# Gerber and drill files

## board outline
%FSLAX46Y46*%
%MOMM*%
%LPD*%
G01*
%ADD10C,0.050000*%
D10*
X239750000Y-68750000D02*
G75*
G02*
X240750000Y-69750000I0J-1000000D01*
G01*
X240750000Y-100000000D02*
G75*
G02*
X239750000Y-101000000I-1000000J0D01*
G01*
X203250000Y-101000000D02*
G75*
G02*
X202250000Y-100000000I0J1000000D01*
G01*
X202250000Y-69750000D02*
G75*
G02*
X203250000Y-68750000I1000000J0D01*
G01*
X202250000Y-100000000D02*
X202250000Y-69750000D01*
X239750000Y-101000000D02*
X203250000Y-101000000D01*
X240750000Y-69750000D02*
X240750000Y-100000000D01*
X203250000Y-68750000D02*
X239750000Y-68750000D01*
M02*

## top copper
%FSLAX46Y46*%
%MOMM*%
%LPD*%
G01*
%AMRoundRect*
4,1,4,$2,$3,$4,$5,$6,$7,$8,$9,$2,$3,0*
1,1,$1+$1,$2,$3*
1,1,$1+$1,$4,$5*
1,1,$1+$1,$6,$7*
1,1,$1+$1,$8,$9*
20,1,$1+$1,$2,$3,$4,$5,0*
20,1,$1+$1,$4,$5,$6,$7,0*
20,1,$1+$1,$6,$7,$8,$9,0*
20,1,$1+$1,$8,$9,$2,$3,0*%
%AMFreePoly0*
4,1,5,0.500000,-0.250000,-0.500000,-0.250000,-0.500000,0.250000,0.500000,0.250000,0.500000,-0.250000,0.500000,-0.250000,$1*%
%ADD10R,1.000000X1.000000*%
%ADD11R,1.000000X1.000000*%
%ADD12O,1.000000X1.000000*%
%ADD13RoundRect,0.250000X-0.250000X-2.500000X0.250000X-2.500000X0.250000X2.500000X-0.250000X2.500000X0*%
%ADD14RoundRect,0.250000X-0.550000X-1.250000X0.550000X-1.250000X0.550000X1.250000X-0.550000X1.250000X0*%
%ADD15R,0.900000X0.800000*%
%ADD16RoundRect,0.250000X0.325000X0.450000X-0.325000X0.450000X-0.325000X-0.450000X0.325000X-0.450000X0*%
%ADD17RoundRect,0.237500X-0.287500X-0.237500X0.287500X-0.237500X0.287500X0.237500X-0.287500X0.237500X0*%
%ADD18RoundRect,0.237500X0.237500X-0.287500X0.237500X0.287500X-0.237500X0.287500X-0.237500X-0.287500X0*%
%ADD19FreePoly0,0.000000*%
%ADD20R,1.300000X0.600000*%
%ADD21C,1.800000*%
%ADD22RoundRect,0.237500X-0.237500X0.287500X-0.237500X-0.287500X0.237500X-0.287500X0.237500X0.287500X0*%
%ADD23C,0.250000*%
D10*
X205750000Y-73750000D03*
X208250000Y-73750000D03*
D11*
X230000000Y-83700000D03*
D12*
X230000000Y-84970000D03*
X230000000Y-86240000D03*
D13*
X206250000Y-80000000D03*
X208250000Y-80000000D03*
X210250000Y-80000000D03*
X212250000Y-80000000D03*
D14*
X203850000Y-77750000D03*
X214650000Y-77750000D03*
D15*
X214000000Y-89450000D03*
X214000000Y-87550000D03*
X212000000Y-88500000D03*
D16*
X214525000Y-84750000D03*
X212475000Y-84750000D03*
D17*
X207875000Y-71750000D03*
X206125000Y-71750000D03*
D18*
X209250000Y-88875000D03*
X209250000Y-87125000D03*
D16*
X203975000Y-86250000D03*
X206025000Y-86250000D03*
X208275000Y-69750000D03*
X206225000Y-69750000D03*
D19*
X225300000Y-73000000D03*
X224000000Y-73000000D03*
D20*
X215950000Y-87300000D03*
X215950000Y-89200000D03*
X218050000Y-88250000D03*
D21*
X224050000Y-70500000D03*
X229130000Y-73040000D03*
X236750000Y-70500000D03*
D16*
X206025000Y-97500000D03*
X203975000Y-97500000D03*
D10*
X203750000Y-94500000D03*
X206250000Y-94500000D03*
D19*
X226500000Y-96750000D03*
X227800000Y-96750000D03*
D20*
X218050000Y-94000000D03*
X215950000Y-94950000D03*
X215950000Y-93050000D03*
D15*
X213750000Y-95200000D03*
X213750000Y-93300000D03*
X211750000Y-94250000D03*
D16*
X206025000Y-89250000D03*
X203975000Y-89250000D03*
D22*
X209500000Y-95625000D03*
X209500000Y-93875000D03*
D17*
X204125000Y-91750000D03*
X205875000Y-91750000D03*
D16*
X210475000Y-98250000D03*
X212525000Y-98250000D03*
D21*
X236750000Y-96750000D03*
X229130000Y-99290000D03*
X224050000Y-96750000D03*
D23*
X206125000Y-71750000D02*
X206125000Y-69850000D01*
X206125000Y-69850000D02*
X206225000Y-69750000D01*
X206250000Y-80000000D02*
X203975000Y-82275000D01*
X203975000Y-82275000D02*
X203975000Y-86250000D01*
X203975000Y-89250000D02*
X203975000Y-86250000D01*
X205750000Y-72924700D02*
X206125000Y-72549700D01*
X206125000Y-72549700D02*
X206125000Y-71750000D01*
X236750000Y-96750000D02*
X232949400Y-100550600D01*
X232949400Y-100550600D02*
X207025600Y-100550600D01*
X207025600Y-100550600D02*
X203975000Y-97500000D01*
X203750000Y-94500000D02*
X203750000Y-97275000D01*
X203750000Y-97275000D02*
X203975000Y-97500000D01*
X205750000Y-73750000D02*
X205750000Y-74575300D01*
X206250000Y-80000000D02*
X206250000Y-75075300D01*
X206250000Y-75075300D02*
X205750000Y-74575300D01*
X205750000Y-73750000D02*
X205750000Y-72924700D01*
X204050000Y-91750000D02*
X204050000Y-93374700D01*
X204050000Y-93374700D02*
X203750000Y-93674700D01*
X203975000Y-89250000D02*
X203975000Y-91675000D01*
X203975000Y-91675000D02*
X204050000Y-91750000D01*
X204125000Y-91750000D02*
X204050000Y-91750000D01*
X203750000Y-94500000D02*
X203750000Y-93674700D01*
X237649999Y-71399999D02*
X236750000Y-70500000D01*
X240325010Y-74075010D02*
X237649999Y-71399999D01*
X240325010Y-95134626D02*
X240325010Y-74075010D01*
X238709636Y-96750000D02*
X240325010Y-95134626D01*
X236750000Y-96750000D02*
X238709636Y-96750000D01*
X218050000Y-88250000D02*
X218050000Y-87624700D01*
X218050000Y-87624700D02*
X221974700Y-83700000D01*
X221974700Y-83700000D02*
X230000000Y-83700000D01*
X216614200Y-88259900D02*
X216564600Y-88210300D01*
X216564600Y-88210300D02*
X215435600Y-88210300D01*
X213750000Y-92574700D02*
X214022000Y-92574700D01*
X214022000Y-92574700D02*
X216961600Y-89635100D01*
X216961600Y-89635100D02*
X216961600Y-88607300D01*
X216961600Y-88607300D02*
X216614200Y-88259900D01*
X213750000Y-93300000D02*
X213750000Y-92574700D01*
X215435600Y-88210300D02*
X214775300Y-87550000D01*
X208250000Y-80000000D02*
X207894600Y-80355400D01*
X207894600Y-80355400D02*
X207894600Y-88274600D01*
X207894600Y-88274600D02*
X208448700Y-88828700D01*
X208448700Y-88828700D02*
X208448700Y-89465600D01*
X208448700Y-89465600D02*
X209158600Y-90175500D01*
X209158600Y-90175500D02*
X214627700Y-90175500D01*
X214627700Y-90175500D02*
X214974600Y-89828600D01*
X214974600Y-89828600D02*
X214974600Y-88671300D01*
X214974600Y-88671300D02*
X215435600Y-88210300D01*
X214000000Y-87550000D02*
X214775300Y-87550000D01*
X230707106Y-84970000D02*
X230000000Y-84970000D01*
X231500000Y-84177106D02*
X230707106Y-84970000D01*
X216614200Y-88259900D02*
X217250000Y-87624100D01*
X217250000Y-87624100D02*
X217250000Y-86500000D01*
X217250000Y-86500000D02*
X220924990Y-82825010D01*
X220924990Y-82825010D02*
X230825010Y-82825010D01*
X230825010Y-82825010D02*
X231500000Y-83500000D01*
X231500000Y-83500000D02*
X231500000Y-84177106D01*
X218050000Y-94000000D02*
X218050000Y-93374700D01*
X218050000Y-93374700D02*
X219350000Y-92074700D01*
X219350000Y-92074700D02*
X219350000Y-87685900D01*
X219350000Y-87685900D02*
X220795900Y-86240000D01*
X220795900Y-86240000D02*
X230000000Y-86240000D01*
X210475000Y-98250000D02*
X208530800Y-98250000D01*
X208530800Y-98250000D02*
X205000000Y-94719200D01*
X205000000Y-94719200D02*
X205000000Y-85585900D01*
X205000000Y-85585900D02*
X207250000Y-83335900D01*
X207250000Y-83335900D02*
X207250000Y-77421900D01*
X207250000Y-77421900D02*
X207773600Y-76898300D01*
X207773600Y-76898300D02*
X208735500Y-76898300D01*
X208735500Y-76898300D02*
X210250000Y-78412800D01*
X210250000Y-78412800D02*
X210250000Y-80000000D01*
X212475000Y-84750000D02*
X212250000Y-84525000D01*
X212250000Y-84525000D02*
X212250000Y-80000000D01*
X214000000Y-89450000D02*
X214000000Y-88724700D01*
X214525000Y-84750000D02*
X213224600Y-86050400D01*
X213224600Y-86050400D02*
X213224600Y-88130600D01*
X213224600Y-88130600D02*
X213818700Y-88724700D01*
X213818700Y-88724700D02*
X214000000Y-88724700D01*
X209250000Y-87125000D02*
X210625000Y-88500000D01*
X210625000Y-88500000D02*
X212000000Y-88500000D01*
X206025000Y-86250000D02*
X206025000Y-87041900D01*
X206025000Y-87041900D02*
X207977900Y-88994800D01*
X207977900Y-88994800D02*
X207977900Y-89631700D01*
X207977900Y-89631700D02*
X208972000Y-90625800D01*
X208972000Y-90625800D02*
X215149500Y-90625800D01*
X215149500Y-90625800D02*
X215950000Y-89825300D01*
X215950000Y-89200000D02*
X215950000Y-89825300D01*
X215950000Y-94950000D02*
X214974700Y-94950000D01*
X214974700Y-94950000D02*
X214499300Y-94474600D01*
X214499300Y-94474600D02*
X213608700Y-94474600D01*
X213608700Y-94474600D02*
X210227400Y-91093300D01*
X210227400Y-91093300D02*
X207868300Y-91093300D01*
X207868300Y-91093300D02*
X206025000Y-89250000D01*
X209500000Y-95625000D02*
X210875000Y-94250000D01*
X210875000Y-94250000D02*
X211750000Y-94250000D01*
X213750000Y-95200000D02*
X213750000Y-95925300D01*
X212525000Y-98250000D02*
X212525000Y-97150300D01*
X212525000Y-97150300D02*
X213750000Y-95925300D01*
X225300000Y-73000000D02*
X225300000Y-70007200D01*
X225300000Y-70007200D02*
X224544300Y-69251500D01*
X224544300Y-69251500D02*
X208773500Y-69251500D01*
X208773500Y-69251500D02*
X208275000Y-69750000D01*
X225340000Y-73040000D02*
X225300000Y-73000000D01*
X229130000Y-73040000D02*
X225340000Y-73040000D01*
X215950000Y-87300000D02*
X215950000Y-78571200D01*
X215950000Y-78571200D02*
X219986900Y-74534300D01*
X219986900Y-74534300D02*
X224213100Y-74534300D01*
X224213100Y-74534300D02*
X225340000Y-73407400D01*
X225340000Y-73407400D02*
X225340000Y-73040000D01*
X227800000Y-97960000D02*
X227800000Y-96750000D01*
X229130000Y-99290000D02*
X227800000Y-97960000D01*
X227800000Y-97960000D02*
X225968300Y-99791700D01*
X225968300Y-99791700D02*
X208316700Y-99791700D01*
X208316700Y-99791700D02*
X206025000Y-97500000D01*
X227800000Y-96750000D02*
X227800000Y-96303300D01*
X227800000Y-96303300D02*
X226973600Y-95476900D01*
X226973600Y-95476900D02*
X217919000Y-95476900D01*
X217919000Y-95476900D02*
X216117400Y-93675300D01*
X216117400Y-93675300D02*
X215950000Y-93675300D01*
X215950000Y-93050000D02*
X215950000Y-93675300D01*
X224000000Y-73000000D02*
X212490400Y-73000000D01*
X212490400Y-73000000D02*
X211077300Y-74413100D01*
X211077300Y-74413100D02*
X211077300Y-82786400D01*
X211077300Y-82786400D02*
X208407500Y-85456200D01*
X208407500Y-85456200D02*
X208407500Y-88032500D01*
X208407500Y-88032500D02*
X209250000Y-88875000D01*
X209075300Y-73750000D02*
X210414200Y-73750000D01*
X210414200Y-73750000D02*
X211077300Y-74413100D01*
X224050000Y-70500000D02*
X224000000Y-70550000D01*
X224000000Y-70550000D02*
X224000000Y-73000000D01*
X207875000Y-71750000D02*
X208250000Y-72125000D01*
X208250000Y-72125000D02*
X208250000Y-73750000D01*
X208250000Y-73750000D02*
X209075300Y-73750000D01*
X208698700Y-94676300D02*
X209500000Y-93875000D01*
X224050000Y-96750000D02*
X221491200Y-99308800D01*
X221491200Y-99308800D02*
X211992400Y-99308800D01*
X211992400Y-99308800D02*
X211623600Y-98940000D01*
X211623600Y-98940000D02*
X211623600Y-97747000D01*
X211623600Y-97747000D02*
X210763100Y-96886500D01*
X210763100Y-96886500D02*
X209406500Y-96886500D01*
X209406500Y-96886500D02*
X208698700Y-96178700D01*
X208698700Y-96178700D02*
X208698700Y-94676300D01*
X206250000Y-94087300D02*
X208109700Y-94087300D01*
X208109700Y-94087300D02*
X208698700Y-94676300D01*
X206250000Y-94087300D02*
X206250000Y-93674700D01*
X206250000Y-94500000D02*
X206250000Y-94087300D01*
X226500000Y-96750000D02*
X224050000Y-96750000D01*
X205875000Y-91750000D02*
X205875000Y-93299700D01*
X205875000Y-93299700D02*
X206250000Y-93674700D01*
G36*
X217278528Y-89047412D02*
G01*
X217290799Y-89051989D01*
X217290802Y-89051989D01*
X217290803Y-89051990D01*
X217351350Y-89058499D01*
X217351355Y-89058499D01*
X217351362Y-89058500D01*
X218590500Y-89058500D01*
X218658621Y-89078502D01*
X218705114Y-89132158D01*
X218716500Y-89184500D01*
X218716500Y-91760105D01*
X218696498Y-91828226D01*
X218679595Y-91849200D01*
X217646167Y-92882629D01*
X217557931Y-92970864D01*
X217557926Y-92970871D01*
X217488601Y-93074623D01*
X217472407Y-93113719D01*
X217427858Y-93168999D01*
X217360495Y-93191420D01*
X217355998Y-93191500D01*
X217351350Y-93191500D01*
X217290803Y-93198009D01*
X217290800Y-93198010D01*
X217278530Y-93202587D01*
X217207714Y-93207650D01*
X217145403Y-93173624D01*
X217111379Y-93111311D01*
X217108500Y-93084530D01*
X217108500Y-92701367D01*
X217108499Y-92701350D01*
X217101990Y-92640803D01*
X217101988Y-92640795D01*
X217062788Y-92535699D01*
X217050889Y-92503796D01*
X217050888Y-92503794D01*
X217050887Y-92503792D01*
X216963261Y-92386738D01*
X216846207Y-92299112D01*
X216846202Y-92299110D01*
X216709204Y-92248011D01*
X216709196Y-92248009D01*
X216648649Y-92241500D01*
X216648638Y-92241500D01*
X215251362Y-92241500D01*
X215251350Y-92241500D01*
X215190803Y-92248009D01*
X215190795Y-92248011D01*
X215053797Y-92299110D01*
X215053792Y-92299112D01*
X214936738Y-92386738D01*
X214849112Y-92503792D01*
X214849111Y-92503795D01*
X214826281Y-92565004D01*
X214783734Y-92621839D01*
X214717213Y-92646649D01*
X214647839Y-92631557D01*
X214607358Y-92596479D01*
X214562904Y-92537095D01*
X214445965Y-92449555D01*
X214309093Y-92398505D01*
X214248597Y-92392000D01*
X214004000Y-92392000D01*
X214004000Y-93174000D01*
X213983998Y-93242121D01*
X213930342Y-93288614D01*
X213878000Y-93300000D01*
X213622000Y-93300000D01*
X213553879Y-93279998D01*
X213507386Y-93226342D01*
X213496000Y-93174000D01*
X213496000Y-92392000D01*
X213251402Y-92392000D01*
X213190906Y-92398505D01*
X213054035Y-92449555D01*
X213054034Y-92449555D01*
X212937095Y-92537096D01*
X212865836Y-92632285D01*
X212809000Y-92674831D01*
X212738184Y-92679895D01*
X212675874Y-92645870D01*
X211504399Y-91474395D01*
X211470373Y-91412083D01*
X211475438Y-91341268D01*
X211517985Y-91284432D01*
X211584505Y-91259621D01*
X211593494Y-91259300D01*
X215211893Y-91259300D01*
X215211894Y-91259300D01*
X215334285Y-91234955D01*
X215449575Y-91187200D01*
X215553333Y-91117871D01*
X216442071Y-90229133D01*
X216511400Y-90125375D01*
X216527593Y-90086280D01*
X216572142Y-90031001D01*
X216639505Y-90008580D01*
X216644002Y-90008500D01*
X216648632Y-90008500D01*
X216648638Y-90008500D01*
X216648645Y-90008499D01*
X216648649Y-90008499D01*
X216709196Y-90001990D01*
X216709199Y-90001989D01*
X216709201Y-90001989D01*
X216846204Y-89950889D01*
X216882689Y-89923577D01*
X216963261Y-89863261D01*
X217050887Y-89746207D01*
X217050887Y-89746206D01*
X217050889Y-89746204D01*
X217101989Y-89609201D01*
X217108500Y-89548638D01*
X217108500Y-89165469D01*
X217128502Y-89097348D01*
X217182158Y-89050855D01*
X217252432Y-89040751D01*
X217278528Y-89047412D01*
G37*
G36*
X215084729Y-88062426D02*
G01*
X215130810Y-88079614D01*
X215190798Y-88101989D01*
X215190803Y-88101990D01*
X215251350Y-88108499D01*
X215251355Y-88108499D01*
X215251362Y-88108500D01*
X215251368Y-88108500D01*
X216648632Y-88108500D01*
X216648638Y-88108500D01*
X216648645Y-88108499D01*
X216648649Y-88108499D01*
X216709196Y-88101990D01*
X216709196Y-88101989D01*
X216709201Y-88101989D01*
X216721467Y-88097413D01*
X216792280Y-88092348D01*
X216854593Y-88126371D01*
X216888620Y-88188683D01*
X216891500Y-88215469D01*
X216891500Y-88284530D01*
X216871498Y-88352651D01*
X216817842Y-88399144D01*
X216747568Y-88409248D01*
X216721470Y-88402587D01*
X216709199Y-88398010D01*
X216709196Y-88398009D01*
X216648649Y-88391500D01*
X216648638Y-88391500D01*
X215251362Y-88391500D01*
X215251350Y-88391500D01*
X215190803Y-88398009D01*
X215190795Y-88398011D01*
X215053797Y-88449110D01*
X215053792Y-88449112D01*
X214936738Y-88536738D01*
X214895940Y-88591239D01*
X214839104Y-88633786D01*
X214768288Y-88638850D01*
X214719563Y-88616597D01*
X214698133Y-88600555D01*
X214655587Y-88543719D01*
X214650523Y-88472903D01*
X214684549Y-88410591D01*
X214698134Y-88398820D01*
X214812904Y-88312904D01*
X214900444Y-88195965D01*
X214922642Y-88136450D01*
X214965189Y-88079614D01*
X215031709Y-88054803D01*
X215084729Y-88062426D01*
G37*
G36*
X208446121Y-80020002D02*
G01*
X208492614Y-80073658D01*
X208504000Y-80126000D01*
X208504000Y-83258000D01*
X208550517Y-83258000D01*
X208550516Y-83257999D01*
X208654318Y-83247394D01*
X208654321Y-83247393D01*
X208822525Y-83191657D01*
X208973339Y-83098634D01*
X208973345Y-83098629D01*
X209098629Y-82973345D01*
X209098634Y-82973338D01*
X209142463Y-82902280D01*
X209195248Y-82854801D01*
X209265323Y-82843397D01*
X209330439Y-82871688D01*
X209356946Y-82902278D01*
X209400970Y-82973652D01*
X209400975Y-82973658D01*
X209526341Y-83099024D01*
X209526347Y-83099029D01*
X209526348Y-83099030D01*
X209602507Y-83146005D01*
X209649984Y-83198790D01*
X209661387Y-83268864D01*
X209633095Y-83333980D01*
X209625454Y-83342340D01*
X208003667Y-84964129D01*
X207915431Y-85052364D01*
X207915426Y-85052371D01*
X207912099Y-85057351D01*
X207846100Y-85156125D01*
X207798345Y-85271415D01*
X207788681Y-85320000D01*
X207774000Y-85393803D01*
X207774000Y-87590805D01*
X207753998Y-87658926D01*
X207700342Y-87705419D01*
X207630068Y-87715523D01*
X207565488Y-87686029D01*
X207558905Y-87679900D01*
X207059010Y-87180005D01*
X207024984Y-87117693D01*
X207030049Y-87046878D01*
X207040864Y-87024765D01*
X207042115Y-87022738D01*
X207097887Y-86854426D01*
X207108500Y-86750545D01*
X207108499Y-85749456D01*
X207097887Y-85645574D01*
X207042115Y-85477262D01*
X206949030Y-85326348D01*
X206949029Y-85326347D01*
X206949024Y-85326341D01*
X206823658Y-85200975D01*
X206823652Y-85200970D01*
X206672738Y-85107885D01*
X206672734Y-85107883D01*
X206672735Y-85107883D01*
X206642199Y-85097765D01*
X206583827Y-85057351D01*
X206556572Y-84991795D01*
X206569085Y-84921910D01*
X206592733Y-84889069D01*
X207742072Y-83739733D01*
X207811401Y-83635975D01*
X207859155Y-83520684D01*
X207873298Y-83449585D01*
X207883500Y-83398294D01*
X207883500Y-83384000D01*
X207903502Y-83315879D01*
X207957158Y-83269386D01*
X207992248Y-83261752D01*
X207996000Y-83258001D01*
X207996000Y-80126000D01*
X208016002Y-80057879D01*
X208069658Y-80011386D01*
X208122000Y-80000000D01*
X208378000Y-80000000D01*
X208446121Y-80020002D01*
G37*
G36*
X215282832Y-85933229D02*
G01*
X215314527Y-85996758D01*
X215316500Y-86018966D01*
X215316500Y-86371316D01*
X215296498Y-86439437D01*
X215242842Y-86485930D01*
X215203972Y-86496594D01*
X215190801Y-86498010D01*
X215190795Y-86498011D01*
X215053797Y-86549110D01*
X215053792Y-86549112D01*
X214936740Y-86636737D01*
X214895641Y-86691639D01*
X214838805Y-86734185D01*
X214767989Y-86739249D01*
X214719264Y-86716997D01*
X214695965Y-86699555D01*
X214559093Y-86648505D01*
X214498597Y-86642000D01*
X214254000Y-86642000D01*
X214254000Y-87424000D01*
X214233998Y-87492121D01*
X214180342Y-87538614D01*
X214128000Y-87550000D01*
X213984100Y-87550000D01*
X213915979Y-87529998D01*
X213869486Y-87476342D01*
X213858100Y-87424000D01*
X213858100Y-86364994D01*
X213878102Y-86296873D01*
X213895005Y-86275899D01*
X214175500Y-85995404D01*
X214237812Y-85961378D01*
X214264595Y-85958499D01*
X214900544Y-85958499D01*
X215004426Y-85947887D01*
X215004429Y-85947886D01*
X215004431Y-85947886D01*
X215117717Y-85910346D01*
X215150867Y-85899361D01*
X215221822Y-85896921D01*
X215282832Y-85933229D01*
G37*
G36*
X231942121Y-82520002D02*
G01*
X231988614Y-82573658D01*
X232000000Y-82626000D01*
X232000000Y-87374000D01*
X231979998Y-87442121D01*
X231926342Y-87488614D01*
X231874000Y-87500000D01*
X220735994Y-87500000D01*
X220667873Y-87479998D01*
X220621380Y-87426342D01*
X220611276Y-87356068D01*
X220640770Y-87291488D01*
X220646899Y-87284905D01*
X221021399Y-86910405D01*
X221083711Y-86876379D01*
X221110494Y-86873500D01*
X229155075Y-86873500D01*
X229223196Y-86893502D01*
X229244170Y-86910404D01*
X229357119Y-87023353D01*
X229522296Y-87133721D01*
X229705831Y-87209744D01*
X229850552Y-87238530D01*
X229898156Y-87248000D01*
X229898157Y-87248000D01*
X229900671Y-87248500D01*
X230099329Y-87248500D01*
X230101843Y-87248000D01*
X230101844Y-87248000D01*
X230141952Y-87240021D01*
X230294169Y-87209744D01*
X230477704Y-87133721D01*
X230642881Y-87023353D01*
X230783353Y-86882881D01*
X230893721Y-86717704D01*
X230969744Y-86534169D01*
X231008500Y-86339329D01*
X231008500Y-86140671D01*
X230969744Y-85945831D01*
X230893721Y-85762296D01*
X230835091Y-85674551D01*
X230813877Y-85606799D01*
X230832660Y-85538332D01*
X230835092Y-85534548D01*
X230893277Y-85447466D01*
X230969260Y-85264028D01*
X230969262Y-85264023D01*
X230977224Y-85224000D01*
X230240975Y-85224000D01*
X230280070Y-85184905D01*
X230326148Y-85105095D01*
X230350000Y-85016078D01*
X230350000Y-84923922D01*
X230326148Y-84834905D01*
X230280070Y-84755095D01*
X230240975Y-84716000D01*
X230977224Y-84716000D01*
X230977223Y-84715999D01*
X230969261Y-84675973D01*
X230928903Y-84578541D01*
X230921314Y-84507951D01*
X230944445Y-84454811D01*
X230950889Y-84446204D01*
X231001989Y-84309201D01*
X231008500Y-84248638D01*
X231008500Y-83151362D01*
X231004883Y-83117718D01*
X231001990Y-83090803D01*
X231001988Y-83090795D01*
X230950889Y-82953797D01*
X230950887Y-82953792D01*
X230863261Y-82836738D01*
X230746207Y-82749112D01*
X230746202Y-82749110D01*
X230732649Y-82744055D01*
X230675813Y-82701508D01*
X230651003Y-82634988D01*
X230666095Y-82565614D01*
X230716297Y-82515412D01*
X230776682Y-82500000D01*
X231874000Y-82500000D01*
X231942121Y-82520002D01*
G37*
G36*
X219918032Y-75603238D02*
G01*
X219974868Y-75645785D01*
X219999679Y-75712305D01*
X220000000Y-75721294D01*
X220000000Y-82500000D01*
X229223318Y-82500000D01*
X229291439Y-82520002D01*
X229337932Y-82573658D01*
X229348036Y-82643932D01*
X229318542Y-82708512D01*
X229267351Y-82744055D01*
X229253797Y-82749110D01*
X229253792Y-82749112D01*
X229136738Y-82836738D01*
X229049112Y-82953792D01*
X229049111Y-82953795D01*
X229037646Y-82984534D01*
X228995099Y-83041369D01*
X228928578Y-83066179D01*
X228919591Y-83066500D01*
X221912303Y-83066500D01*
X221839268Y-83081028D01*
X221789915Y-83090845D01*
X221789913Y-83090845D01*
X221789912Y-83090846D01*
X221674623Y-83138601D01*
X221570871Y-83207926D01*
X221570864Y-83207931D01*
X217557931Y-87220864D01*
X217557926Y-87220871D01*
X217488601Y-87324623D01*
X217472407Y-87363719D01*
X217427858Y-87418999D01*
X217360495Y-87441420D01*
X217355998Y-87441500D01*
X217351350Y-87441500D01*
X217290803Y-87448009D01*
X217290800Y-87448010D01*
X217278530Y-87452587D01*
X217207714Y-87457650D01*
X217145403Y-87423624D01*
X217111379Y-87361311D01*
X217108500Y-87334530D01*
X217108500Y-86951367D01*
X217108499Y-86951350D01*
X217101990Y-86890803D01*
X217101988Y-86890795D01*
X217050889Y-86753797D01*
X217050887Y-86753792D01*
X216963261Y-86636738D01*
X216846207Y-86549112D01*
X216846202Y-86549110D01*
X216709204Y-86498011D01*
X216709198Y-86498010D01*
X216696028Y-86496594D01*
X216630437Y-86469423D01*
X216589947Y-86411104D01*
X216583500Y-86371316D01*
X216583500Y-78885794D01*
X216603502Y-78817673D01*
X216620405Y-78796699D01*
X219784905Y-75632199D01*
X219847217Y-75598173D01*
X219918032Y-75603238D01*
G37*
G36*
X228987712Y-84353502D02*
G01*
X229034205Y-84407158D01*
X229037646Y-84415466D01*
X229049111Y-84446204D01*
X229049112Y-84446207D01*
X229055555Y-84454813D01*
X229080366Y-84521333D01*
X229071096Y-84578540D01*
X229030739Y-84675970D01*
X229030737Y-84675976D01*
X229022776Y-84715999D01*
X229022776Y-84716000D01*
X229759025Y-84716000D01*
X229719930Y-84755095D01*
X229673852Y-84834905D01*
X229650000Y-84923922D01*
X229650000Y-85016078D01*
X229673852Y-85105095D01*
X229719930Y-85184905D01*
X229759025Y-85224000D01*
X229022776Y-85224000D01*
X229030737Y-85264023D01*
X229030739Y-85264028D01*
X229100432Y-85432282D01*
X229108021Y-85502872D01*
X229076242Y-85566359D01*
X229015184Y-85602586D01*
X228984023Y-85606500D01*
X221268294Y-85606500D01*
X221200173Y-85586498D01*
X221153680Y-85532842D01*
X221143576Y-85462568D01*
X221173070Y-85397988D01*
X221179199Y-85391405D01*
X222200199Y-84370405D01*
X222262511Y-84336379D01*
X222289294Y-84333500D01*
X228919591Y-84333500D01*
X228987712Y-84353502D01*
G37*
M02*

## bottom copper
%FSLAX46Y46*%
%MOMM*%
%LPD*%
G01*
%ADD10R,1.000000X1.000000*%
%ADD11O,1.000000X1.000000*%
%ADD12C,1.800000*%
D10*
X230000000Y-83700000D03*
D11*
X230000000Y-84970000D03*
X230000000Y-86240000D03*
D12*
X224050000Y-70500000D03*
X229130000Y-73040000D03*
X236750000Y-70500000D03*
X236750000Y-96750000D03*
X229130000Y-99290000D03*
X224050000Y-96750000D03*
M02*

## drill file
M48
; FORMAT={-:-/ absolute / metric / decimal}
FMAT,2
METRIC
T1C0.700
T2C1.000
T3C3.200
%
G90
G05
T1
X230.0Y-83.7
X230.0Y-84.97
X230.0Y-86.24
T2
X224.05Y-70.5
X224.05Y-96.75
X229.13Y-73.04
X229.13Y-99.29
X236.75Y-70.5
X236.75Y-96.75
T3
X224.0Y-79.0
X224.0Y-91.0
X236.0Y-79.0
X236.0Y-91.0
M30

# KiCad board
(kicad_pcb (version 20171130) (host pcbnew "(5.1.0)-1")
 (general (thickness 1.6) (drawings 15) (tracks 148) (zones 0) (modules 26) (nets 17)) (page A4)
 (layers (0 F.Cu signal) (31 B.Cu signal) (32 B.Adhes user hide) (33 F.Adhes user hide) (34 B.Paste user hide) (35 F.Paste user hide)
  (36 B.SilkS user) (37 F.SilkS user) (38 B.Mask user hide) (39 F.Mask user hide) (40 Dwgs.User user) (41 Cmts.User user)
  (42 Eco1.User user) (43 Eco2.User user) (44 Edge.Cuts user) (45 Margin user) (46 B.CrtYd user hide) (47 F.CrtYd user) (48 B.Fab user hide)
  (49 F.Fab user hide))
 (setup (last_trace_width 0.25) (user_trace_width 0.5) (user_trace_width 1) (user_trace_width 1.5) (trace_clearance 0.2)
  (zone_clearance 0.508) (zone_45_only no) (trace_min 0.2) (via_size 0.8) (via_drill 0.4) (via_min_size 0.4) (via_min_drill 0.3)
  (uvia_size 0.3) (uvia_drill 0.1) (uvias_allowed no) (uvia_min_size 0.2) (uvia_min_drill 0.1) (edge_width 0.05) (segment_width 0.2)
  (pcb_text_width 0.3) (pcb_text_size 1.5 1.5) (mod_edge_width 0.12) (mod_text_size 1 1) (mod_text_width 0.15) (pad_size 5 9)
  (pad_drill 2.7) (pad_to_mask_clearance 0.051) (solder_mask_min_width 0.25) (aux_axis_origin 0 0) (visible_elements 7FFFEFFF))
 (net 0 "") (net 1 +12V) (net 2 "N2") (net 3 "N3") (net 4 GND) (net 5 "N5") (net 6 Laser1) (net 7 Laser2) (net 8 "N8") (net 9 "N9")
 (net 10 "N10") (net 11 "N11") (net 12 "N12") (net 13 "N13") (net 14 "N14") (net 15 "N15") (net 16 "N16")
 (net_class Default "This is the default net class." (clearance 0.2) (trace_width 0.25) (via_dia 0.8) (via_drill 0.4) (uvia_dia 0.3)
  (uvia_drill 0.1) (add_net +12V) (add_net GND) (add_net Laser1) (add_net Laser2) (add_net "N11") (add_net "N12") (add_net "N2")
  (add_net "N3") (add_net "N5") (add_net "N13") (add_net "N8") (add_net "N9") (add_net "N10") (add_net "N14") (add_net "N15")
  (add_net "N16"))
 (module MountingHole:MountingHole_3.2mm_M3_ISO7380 (layer F.Cu) (at 224 79)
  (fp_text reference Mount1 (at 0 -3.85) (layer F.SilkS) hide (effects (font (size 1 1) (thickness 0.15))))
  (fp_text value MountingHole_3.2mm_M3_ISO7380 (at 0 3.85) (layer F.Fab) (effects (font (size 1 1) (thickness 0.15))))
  (pad 1 np_thru_hole circle (at 0 0) (size 3.2 3.2) (drill 3.2) (layers *.Cu *.Mask)))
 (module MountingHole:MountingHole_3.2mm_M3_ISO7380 (layer F.Cu) (at 236 79)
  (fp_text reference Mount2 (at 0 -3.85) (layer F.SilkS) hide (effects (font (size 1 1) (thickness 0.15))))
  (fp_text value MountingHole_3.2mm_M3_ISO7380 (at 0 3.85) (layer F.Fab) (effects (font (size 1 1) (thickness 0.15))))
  (pad 1 np_thru_hole circle (at 0 0) (size 3.2 3.2) (drill 3.2) (layers *.Cu *.Mask)))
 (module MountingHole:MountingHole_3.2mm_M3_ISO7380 (layer F.Cu) (at 236 91)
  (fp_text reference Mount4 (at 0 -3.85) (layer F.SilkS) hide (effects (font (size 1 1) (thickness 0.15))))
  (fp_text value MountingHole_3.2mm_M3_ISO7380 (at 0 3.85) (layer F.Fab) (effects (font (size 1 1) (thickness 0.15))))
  (pad 1 np_thru_hole circle (at 0 0) (size 3.2 3.2) (drill 3.2) (layers *.Cu *.Mask)))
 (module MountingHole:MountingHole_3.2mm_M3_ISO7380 (layer F.Cu) (at 224 91)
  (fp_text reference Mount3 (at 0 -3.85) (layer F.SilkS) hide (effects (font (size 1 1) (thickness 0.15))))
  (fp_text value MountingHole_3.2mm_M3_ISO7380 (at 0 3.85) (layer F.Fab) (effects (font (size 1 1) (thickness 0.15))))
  (pad 1 np_thru_hole circle (at 0 0) (size 3.2 3.2) (drill 3.2) (layers *.Cu *.Mask)))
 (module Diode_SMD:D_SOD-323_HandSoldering (layer F.Cu) (at 207 73.75)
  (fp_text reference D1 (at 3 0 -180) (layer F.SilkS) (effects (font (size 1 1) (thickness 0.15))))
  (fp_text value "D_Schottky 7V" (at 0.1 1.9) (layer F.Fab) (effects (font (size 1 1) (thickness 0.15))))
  (pad 1 smd rect (at -1.25 0) (size 1 1) (layers F.Cu F.Paste F.Mask) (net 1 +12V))
  (pad 2 smd rect (at 1.25 0) (size 1 1) (layers F.Cu F.Paste F.Mask) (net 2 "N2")))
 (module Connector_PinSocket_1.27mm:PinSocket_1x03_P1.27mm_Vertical (layer F.Cu) (at 230 83.7)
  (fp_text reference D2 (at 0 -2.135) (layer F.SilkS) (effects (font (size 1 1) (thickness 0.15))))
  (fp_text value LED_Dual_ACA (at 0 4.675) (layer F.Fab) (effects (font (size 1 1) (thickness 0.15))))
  (pad 1 thru_hole rect (at 0 0) (size 1 1) (drill 0.7) (layers *.Cu *.Mask) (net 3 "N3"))
  (pad 2 thru_hole oval (at 0 1.27) (size 1 1) (drill 0.7) (layers *.Cu *.Mask) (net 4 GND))
  (pad 3 thru_hole oval (at 0 2.54) (size 1 1) (drill 0.7) (layers *.Cu *.Mask) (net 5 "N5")))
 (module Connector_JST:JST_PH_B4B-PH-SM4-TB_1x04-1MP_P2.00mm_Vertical (layer F.Cu) (at 209.25 79.5)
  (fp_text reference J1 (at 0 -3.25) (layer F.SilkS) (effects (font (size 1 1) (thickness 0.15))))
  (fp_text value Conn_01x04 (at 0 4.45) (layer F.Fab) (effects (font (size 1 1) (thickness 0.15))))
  (pad 1 smd roundrect (at -3 0.5) (size 1 5.5) (layers F.Cu F.Paste F.Mask) (roundrect_rratio 0.25) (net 1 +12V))
  (pad 2 smd roundrect (at -1 0.5) (size 1 5.5) (layers F.Cu F.Paste F.Mask) (roundrect_rratio 0.25) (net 4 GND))
  (pad 3 smd roundrect (at 1 0.5) (size 1 5.5) (layers F.Cu F.Paste F.Mask) (roundrect_rratio 0.25) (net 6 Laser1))
  (pad 4 smd roundrect (at 3 0.5) (size 1 5.5) (layers F.Cu F.Paste F.Mask) (roundrect_rratio 0.25) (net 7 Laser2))
  (pad MP smd roundrect (at -5.4 -1.75) (size 1.6 3) (layers F.Cu F.Paste F.Mask) (roundrect_rratio 0.15625))
  (pad MP smd roundrect (at 5.4 -1.75) (size 1.6 3) (layers F.Cu F.Paste F.Mask) (roundrect_rratio 0.15625)))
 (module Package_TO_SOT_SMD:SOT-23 (layer F.Cu) (at 213 88.5 180)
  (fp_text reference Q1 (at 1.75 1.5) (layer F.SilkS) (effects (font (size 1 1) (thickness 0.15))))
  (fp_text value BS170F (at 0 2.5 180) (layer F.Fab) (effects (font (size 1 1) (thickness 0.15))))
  (pad 1 smd rect (at -1 -0.95 180) (size 0.9 0.8) (layers F.Cu F.Paste F.Mask) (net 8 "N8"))
  (pad 2 smd rect (at -1 0.95 180) (size 0.9 0.8) (layers F.Cu F.Paste F.Mask) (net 4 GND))
  (pad 3 smd rect (at 1 0 180) (size 0.9 0.8) (layers F.Cu F.Paste F.Mask) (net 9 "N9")))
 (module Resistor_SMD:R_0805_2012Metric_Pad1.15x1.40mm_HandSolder (layer F.Cu) (at 213.5 84.75 180)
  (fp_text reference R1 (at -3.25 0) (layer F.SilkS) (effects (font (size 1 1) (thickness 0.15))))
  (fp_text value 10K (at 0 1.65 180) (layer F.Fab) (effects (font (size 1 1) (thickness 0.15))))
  (pad 1 smd roundrect (at -1.025 0 180) (size 1.15 1.4) (layers F.Cu F.Paste F.Mask) (roundrect_rratio 0.217391) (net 8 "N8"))
  (pad 2 smd roundrect (at 1.025 0 180) (size 1.15 1.4) (layers F.Cu F.Paste F.Mask) (roundrect_rratio 0.217391) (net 7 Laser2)))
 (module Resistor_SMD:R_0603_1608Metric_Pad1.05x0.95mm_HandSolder (layer F.Cu) (at 207 71.75)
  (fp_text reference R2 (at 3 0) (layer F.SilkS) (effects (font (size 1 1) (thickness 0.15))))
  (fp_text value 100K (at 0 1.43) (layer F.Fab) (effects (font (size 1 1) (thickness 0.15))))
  (pad 2 smd roundrect (at 0.875 0) (size 1.05 0.95) (layers F.Cu F.Paste F.Mask) (roundrect_rratio 0.25) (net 2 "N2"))
  (pad 1 smd roundrect (at -0.875 0) (size 1.05 0.95) (layers F.Cu F.Paste F.Mask) (roundrect_rratio 0.25) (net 1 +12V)))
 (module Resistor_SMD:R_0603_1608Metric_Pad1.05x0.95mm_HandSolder (layer F.Cu) (at 209.25 88 90)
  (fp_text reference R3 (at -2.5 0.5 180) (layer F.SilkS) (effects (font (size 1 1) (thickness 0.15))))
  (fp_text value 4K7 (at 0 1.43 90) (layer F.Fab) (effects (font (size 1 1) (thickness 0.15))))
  (pad 1 smd roundrect (at -0.875 0 90) (size 1.05 0.95) (layers F.Cu F.Paste F.Mask) (roundrect_rratio 0.25) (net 2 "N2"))
  (pad 2 smd roundrect (at 0.875 0 90) (size 1.05 0.95) (layers F.Cu F.Paste F.Mask) (roundrect_rratio 0.25) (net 9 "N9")))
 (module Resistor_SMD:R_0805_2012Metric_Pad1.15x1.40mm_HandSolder (layer F.Cu) (at 205 86.25 180)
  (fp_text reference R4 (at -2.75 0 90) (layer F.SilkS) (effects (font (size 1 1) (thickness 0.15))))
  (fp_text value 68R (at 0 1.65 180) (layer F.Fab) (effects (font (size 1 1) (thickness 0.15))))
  (pad 2 smd roundrect (at 1.025 0 180) (size 1.15 1.4) (layers F.Cu F.Paste F.Mask) (roundrect_rratio 0.217391) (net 1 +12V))
  (pad 1 smd roundrect (at -1.025 0 180) (size 1.15 1.4) (layers F.Cu F.Paste F.Mask) (roundrect_rratio 0.217391) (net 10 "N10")))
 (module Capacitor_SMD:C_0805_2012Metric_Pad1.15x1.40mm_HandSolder (layer F.Cu) (at 207.25 69.75 180)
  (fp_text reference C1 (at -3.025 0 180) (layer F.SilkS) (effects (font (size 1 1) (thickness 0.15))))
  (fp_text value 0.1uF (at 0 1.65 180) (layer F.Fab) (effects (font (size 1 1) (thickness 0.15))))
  (pad 1 smd roundrect (at -1.025 0 180) (size 1.15 1.4) (layers F.Cu F.Paste F.Mask) (roundrect_rratio 0.217391) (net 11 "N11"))
  (pad 2 smd roundrect (at 1.025 0 180) (size 1.15 1.4) (layers F.Cu F.Paste F.Mask) (roundrect_rratio 0.217391) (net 1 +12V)))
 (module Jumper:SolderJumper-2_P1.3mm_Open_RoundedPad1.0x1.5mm (layer F.Cu) (at 224.65 73)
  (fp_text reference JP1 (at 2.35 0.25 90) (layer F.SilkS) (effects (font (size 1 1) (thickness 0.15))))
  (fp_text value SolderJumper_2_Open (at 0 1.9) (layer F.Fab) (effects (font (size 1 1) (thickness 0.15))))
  (pad 2 smd custom (at 0.65 0) (size 1 0.5) (layers F.Cu F.Mask) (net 11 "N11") (zone_connect 2)
   (options (clearance outline) (anchor rect)) (primitives))
  (pad 1 smd custom (at -0.65 0) (size 1 0.5) (layers F.Cu F.Mask) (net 2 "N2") (zone_connect 2) (options (clearance outline) (anchor rect))
   (primitives)))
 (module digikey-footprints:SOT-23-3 (layer F.Cu) (at 217 88.25)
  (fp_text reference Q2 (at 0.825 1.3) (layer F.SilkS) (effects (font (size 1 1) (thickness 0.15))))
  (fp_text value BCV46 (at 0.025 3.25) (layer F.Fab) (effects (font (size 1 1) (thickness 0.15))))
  (pad 1 smd rect (at -1.05 -0.95) (size 1.3 0.6) (layers F.Cu F.Paste F.Mask) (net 11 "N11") (solder_mask_margin 0.07))
  (pad 2 smd rect (at -1.05 0.95) (size 1.3 0.6) (layers F.Cu F.Paste F.Mask) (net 10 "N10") (solder_mask_margin 0.07))
  (pad 3 smd rect (at 1.05 0) (size 1.3 0.6) (layers F.Cu F.Paste F.Mask) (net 3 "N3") (solder_mask_margin 0.07)))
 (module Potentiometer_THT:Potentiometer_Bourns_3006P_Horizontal (layer B.Cu) (at 236.75 70.5)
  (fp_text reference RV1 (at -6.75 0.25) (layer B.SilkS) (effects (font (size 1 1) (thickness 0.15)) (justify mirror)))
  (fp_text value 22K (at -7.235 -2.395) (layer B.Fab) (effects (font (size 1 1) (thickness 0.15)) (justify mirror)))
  (pad 3 thru_hole circle (at -12.7 0) (size 1.8 1.8) (drill 1) (layers *.Cu *.Mask) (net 2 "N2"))
  (pad 2 thru_hole circle (at -7.62 2.54) (size 1.8 1.8) (drill 1) (layers *.Cu *.Mask) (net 11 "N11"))
  (pad 1 thru_hole circle (at 0 0) (size 1.8 1.8) (drill 1) (layers *.Cu *.Mask) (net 1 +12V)))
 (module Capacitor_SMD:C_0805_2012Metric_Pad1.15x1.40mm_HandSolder (layer F.Cu) (at 205 97.5 180)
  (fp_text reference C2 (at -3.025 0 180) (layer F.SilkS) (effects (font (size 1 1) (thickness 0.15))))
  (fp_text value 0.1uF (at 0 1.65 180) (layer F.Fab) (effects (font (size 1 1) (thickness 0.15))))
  (pad 1 smd roundrect (at -1.025 0 180) (size 1.15 1.4) (layers F.Cu F.Paste F.Mask) (roundrect_rratio 0.217391) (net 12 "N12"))
  (pad 2 smd roundrect (at 1.025 0 180) (size 1.15 1.4) (layers F.Cu F.Paste F.Mask) (roundrect_rratio 0.217391) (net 1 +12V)))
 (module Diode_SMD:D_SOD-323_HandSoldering (layer F.Cu) (at 205 94.5)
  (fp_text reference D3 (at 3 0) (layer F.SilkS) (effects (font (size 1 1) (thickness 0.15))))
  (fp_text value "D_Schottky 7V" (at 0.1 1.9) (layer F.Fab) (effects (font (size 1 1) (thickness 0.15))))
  (pad 1 smd rect (at -1.25 0) (size 1 1) (layers F.Cu F.Paste F.Mask) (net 1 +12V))
  (pad 2 smd rect (at 1.25 0) (size 1 1) (layers F.Cu F.Paste F.Mask) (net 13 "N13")))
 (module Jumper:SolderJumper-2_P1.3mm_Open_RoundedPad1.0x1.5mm (layer F.Cu) (at 227.15 96.75)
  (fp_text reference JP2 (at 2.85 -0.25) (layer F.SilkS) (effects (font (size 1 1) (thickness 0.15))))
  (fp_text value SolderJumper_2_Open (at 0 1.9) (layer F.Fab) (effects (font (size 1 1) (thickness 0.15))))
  (pad 1 smd custom (at -0.65 0) (size 1 0.5) (layers F.Cu F.Mask) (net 13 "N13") (zone_connect 2)
   (options (clearance outline) (anchor rect)) (primitives))
  (pad 2 smd custom (at 0.65 0) (size 1 0.5) (layers F.Cu F.Mask) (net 12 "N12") (zone_connect 2)
   (options (clearance outline) (anchor rect)) (primitives)))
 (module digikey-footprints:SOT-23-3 (layer F.Cu) (at 217 94)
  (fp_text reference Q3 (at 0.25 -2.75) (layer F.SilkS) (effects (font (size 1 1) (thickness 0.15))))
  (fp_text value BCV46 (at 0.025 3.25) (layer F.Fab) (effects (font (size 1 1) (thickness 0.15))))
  (pad 3 smd rect (at 1.05 0) (size 1.3 0.6) (layers F.Cu F.Paste F.Mask) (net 5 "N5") (solder_mask_margin 0.07))
  (pad 2 smd rect (at -1.05 0.95) (size 1.3 0.6) (layers F.Cu F.Paste F.Mask) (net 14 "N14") (solder_mask_margin 0.07))
  (pad 1 smd rect (at -1.05 -0.95) (size 1.3 0.6) (layers F.Cu F.Paste F.Mask) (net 12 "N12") (solder_mask_margin 0.07)))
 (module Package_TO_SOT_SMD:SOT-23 (layer F.Cu) (at 212.75 94.25 180)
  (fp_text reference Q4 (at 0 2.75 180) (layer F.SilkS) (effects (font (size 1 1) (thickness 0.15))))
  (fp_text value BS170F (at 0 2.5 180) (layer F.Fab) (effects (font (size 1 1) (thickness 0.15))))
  (pad 1 smd rect (at -1 -0.95 180) (size 0.9 0.8) (layers F.Cu F.Paste F.Mask) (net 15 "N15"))
  (pad 2 smd rect (at -1 0.95 180) (size 0.9 0.8) (layers F.Cu F.Paste F.Mask) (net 4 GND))
  (pad 3 smd rect (at 1 0 180) (size 0.9 0.8) (layers F.Cu F.Paste F.Mask) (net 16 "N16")))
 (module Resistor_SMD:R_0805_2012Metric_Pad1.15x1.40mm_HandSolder (layer F.Cu) (at 205 89.25 180)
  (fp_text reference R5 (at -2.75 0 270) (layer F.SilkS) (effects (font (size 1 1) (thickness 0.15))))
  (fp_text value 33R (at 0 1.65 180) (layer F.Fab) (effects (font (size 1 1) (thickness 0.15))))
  (pad 1 smd roundrect (at -1.025 0 180) (size 1.15 1.4) (layers F.Cu F.Paste F.Mask) (roundrect_rratio 0.217391) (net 14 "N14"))
  (pad 2 smd roundrect (at 1.025 0 180) (size 1.15 1.4) (layers F.Cu F.Paste F.Mask) (roundrect_rratio 0.217391) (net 1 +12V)))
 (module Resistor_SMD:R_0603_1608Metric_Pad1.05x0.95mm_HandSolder (layer F.Cu) (at 209.5 94.75 270)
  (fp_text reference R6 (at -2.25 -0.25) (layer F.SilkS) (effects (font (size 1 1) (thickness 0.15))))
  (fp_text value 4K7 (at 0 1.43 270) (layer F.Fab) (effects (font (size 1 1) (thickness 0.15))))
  (pad 2 smd roundrect (at 0.875 0 270) (size 1.05 0.95) (layers F.Cu F.Paste F.Mask) (roundrect_rratio 0.25) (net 16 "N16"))
  (pad 1 smd roundrect (at -0.875 0 270) (size 1.05 0.95) (layers F.Cu F.Paste F.Mask) (roundrect_rratio 0.25) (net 13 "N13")))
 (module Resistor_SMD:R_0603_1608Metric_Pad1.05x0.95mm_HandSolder (layer F.Cu) (at 205 91.75)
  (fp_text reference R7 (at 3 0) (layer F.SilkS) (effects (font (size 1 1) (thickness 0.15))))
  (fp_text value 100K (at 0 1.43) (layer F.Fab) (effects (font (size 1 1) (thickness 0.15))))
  (pad 1 smd roundrect (at -0.875 0) (size 1.05 0.95) (layers F.Cu F.Paste F.Mask) (roundrect_rratio 0.25) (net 1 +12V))
  (pad 2 smd roundrect (at 0.875 0) (size 1.05 0.95) (layers F.Cu F.Paste F.Mask) (roundrect_rratio 0.25) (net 13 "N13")))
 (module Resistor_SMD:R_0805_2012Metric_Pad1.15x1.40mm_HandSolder (layer F.Cu) (at 211.5 98.25 180)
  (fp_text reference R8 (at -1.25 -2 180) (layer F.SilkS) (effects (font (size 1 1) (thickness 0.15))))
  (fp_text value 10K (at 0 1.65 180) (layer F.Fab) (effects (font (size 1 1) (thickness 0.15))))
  (pad 2 smd roundrect (at 1.025 0 180) (size 1.15 1.4) (layers F.Cu F.Paste F.Mask) (roundrect_rratio 0.217391) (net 6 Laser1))
  (pad 1 smd roundrect (at -1.025 0 180) (size 1.15 1.4) (layers F.Cu F.Paste F.Mask) (roundrect_rratio 0.217391) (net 15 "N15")))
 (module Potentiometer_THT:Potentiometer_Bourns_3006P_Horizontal (layer B.Cu) (at 236.75 96.75)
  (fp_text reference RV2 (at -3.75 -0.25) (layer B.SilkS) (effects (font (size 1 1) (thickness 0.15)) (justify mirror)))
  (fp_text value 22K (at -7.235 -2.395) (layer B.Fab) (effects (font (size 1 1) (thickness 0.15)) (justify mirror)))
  (pad 1 thru_hole circle (at 0 0) (size 1.8 1.8) (drill 1) (layers *.Cu *.Mask) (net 1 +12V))
  (pad 2 thru_hole circle (at -7.62 2.54) (size 1.8 1.8) (drill 1) (layers *.Cu *.Mask) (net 12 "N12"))
  (pad 3 thru_hole circle (at -12.7 0) (size 1.8 1.8) (drill 1) (layers *.Cu *.Mask) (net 13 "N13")))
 (gr_arc (start 239.75 69.75) (end 240.75 69.75) (angle -90) (layer Edge.Cuts) (width 0.05))
 (gr_arc (start 239.75 100) (end 239.75 101) (angle -90) (layer Edge.Cuts) (width 0.05))
 (gr_arc (start 203.25 100) (end 202.25 100) (angle -90) (layer Edge.Cuts) (width 0.05))
 (gr_arc (start 203.25 69.75) (end 203.25 68.75) (angle -90) (layer Edge.Cuts) (width 0.05))
 (gr_line (start 202.25 100) (end 202.25 69.75) (layer Edge.Cuts) (width 0.05))
 (gr_line (start 239.75 101) (end 203.25 101) (layer Edge.Cuts) (width 0.05))
 (gr_line (start 240.75 69.75) (end 240.75 100) (layer Edge.Cuts) (width 0.05))
 (gr_line (start 203.25 68.75) (end 239.75 68.75) (layer Edge.Cuts) (width 0.05))
 (segment (start 206.125 71.75) (end 206.125 69.85) (width 0.25) (layer F.Cu) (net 1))
 (segment (start 206.125 69.85) (end 206.225 69.75) (width 0.25) (layer F.Cu) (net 1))
 (segment (start 206.25 80) (end 203.975 82.275) (width 0.25) (layer F.Cu) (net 1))
 (segment (start 203.975 82.275) (end 203.975 86.25) (width 0.25) (layer F.Cu) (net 1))
 (segment (start 203.975 89.25) (end 203.975 86.25) (width 0.25) (layer F.Cu) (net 1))
 (segment (start 205.75 72.9247) (end 206.125 72.5497) (width 0.25) (layer F.Cu) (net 1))
 (segment (start 206.125 72.5497) (end 206.125 71.75) (width 0.25) (layer F.Cu) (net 1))
 (segment (start 236.75 96.75) (end 232.9494 100.5506) (width 0.25) (layer F.Cu) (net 1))
 (segment (start 232.9494 100.5506) (end 207.0256 100.5506) (width 0.25) (layer F.Cu) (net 1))
 (segment (start 207.0256 100.5506) (end 203.975 97.5) (width 0.25) (layer F.Cu) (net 1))
 (segment (start 203.75 94.5) (end 203.75 97.275) (width 0.25) (layer F.Cu) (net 1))
 (segment (start 203.75 97.275) (end 203.975 97.5) (width 0.25) (layer F.Cu) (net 1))
 (segment (start 205.75 73.75) (end 205.75 74.5753) (width 0.25) (layer F.Cu) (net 1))
 (segment (start 206.25 80) (end 206.25 75.0753) (width 0.25) (layer F.Cu) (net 1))
 (segment (start 206.25 75.0753) (end 205.75 74.5753) (width 0.25) (layer F.Cu) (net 1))
 (segment (start 205.75 73.75) (end 205.75 72.9247) (width 0.25) (layer F.Cu) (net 1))
 (segment (start 204.05 91.75) (end 204.05 93.3747) (width 0.25) (layer F.Cu) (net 1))
 (segment (start 204.05 93.3747) (end 203.75 93.6747) (width 0.25) (layer F.Cu) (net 1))
 (segment (start 203.975 89.25) (end 203.975 91.675) (width 0.25) (layer F.Cu) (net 1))
 (segment (start 203.975 91.675) (end 204.05 91.75) (width 0.25) (layer F.Cu) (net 1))
 (segment (start 204.125 91.75) (end 204.05 91.75) (width 0.25) (layer F.Cu) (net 1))
 (segment (start 203.75 94.5) (end 203.75 93.6747) (width 0.25) (layer F.Cu) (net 1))
 (segment (start 237.649999 71.399999) (end 236.75 70.5) (width 0.25) (layer F.Cu) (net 1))
 (segment (start 240.32501 74.07501) (end 237.649999 71.399999) (width 0.25) (layer F.Cu) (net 1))
 (segment (start 240.32501 95.134626) (end 240.32501 74.07501) (width 0.25) (layer F.Cu) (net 1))
 (segment (start 238.709636 96.75) (end 240.32501 95.134626) (width 0.25) (layer F.Cu) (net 1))
 (segment (start 236.75 96.75) (end 238.709636 96.75) (width 0.25) (layer F.Cu) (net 1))
 (segment (start 218.05 88.25) (end 218.05 87.6247) (width 0.25) (layer F.Cu) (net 3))
 (segment (start 218.05 87.6247) (end 221.9747 83.7) (width 0.25) (layer F.Cu) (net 3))
 (segment (start 221.9747 83.7) (end 230 83.7) (width 0.25) (layer F.Cu) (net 3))
 (segment (start 216.6142 88.2599) (end 216.5646 88.2103) (width 0.25) (layer F.Cu) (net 4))
 (segment (start 216.5646 88.2103) (end 215.4356 88.2103) (width 0.25) (layer F.Cu) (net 4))
 (segment (start 213.75 92.5747) (end 214.022 92.5747) (width 0.25) (layer F.Cu) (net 4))
 (segment (start 214.022 92.5747) (end 216.9616 89.6351) (width 0.25) (layer F.Cu) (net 4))
 (segment (start 216.9616 89.6351) (end 216.9616 88.6073) (width 0.25) (layer F.Cu) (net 4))
 (segment (start 216.9616 88.6073) (end 216.6142 88.2599) (width 0.25) (layer F.Cu) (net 4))
 (segment (start 213.75 93.3) (end 213.75 92.5747) (width 0.25) (layer F.Cu) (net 4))
 (segment (start 215.4356 88.2103) (end 214.7753 87.55) (width 0.25) (layer F.Cu) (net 4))
 (segment (start 208.25 80) (end 207.8946 80.3554) (width 0.25) (layer F.Cu) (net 4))
 (segment (start 207.8946 80.3554) (end 207.8946 88.2746) (width 0.25) (layer F.Cu) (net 4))
 (segment (start 207.8946 88.2746) (end 208.4487 88.8287) (width 0.25) (layer F.Cu) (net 4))
 (segment (start 208.4487 88.8287) (end 208.4487 89.4656) (width 0.25) (layer F.Cu) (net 4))
 (segment (start 208.4487 89.4656) (end 209.1586 90.1755) (width 0.25) (layer F.Cu) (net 4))
 (segment (start 209.1586 90.1755) (end 214.6277 90.1755) (width 0.25) (layer F.Cu) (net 4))
 (segment (start 214.6277 90.1755) (end 214.9746 89.8286) (width 0.25) (layer F.Cu) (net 4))
 (segment (start 214.9746 89.8286) (end 214.9746 88.6713) (width 0.25) (layer F.Cu) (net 4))
 (segment (start 214.9746 88.6713) (end 215.4356 88.2103) (width 0.25) (layer F.Cu) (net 4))
 (segment (start 214 87.55) (end 214.7753 87.55) (width 0.25) (layer F.Cu) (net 4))
 (segment (start 230.707106 84.97) (end 230 84.97) (width 0.25) (layer F.Cu) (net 4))
 (segment (start 231.5 84.177106) (end 230.707106 84.97) (width 0.25) (layer F.Cu) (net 4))
 (segment (start 216.6142 88.2599) (end 217.25 87.6241) (width 0.25) (layer F.Cu) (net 4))
 (segment (start 217.25 87.6241) (end 217.25 86.5) (width 0.25) (layer F.Cu) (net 4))
 (segment (start 217.25 86.5) (end 220.92499 82.82501) (width 0.25) (layer F.Cu) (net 4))
 (segment (start 220.92499 82.82501) (end 230.82501 82.82501) (width 0.25) (layer F.Cu) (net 4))
 (segment (start 230.82501 82.82501) (end 231.5 83.5) (width 0.25) (layer F.Cu) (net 4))
 (segment (start 231.5 83.5) (end 231.5 84.177106) (width 0.25) (layer F.Cu) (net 4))
 (segment (start 218.05 94) (end 218.05 93.3747) (width 0.25) (layer F.Cu) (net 5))
 (segment (start 218.05 93.3747) (end 219.35 92.0747) (width 0.25) (layer F.Cu) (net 5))
 (segment (start 219.35 92.0747) (end 219.35 87.6859) (width 0.25) (layer F.Cu) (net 5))
 (segment (start 219.35 87.6859) (end 220.7959 86.24) (width 0.25) (layer F.Cu) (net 5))
 (segment (start 220.7959 86.24) (end 230 86.24) (width 0.25) (layer F.Cu) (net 5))
 (segment (start 210.475 98.25) (end 208.5308 98.25) (width 0.25) (layer F.Cu) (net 6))
 (segment (start 208.5308 98.25) (end 205 94.7192) (width 0.25) (layer F.Cu) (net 6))
 (segment (start 205 94.7192) (end 205 85.5859) (width 0.25) (layer F.Cu) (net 6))
 (segment (start 205 85.5859) (end 207.25 83.3359) (width 0.25) (layer F.Cu) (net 6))
 (segment (start 207.25 83.3359) (end 207.25 77.4219) (width 0.25) (layer F.Cu) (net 6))
 (segment (start 207.25 77.4219) (end 207.7736 76.8983) (width 0.25) (layer F.Cu) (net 6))
 (segment (start 207.7736 76.8983) (end 208.7355 76.8983) (width 0.25) (layer F.Cu) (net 6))
 (segment (start 208.7355 76.8983) (end 210.25 78.4128) (width 0.25) (layer F.Cu) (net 6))
 (segment (start 210.25 78.4128) (end 210.25 80) (width 0.25) (layer F.Cu) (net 6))
 (segment (start 212.475 84.75) (end 212.25 84.525) (width 0.25) (layer F.Cu) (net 7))
 (segment (start 212.25 84.525) (end 212.25 80) (width 0.25) (layer F.Cu) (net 7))
 (segment (start 214 89.45) (end 214 88.7247) (width 0.25) (layer F.Cu) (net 8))
 (segment (start 214.525 84.75) (end 213.2246 86.0504) (width 0.25) (layer F.Cu) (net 8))
 (segment (start 213.2246 86.0504) (end 213.2246 88.1306) (width 0.25) (layer F.Cu) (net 8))
 (segment (start 213.2246 88.1306) (end 213.8187 88.7247) (width 0.25) (layer F.Cu) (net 8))
 (segment (start 213.8187 88.7247) (end 214 88.7247) (width 0.25) (layer F.Cu) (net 8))
 (segment (start 209.25 87.125) (end 210.625 88.5) (width 0.25) (layer F.Cu) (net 9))
 (segment (start 210.625 88.5) (end 212 88.5) (width 0.25) (layer F.Cu) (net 9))
 (segment (start 206.025 86.25) (end 206.025 87.0419) (width 0.25) (layer F.Cu) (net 10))
 (segment (start 206.025 87.0419) (end 207.9779 88.9948) (width 0.25) (layer F.Cu) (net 10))
 (segment (start 207.9779 88.9948) (end 207.9779 89.6317) (width 0.25) (layer F.Cu) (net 10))
 (segment (start 207.9779 89.6317) (end 208.972 90.6258) (width 0.25) (layer F.Cu) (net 10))
 (segment (start 208.972 90.6258) (end 215.1495 90.6258) (width 0.25) (layer F.Cu) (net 10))
 (segment (start 215.1495 90.6258) (end 215.95 89.8253) (width 0.25) (layer F.Cu) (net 10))
 (segment (start 215.95 89.2) (end 215.95 89.8253) (width 0.25) (layer F.Cu) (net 10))
 (segment (start 215.95 94.95) (end 214.9747 94.95) (width 0.25) (layer F.Cu) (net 14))
 (segment (start 214.9747 94.95) (end 214.4993 94.4746) (width 0.25) (layer F.Cu) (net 14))
 (segment (start 214.4993 94.4746) (end 213.6087 94.4746) (width 0.25) (layer F.Cu) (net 14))
 (segment (start 213.6087 94.4746) (end 210.2274 91.0933) (width 0.25) (layer F.Cu) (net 14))
 (segment (start 210.2274 91.0933) (end 207.8683 91.0933) (width 0.25) (layer F.Cu) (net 14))
 (segment (start 207.8683 91.0933) (end 206.025 89.25) (width 0.25) (layer F.Cu) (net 14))
 (segment (start 209.5 95.625) (end 210.875 94.25) (width 0.25) (layer F.Cu) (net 16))
 (segment (start 210.875 94.25) (end 211.75 94.25) (width 0.25) (layer F.Cu) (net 16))
 (segment (start 213.75 95.2) (end 213.75 95.9253) (width 0.25) (layer F.Cu) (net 15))
 (segment (start 212.525 98.25) (end 212.525 97.1503) (width 0.25) (layer F.Cu) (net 15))
 (segment (start 212.525 97.1503) (end 213.75 95.9253) (width 0.25) (layer F.Cu) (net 15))
 (segment (start 225.3 73) (end 225.3 70.0072) (width 0.25) (layer F.Cu) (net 11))
 (segment (start 225.3 70.0072) (end 224.5443 69.2515) (width 0.25) (layer F.Cu) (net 11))
 (segment (start 224.5443 69.2515) (end 208.7735 69.2515) (width 0.25) (layer F.Cu) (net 11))
 (segment (start 208.7735 69.2515) (end 208.275 69.75) (width 0.25) (layer F.Cu) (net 11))
 (segment (start 225.34 73.04) (end 225.3 73) (width 0.25) (layer F.Cu) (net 11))
 (segment (start 229.13 73.04) (end 225.34 73.04) (width 0.25) (layer F.Cu) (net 11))
 (segment (start 215.95 87.3) (end 215.95 78.5712) (width 0.25) (layer F.Cu) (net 11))
 (segment (start 215.95 78.5712) (end 219.9869 74.5343) (width 0.25) (layer F.Cu) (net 11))
 (segment (start 219.9869 74.5343) (end 224.2131 74.5343) (width 0.25) (layer F.Cu) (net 11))
 (segment (start 224.2131 74.5343) (end 225.34 73.4074) (width 0.25) (layer F.Cu) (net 11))
 (segment (start 225.34 73.4074) (end 225.34 73.04) (width 0.25) (layer F.Cu) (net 11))
 (segment (start 227.8 97.96) (end 227.8 96.75) (width 0.25) (layer F.Cu) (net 12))
 (segment (start 229.13 99.29) (end 227.8 97.96) (width 0.25) (layer F.Cu) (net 12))
 (segment (start 227.8 97.96) (end 225.9683 99.7917) (width 0.25) (layer F.Cu) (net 12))
 (segment (start 225.9683 99.7917) (end 208.3167 99.7917) (width 0.25) (layer F.Cu) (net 12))
 (segment (start 208.3167 99.7917) (end 206.025 97.5) (width 0.25) (layer F.Cu) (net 12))
 (segment (start 227.8 96.75) (end 227.8 96.3033) (width 0.25) (layer F.Cu) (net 12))
 (segment (start 227.8 96.3033) (end 226.9736 95.4769) (width 0.25) (layer F.Cu) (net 12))
 (segment (start 226.9736 95.4769) (end 217.919 95.4769) (width 0.25) (layer F.Cu) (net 12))
 (segment (start 217.919 95.4769) (end 216.1174 93.6753) (width 0.25) (layer F.Cu) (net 12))
 (segment (start 216.1174 93.6753) (end 215.95 93.6753) (width 0.25) (layer F.Cu) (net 12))
 (segment (start 215.95 93.05) (end 215.95 93.6753) (width 0.25) (layer F.Cu) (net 12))
 (segment (start 224 73) (end 212.4904 73) (width 0.25) (layer F.Cu) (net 2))
 (segment (start 212.4904 73) (end 211.0773 74.4131) (width 0.25) (layer F.Cu) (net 2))
 (segment (start 211.0773 74.4131) (end 211.0773 82.7864) (width 0.25) (layer F.Cu) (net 2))
 (segment (start 211.0773 82.7864) (end 208.4075 85.4562) (width 0.25) (layer F.Cu) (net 2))
 (segment (start 208.4075 85.4562) (end 208.4075 88.0325) (width 0.25) (layer F.Cu) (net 2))
 (segment (start 208.4075 88.0325) (end 209.25 88.875) (width 0.25) (layer F.Cu) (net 2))
 (segment (start 209.0753 73.75) (end 210.4142 73.75) (width 0.25) (layer F.Cu) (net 2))
 (segment (start 210.4142 73.75) (end 211.0773 74.4131) (width 0.25) (layer F.Cu) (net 2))
 (segment (start 224.05 70.5) (end 224 70.55) (width 0.25) (layer F.Cu) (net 2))
 (segment (start 224 70.55) (end 224 73) (width 0.25) (layer F.Cu) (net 2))
 (segment (start 207.875 71.75) (end 208.25 72.125) (width 0.25) (layer F.Cu) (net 2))
 (segment (start 208.25 72.125) (end 208.25 73.75) (width 0.25) (layer F.Cu) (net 2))
 (segment (start 208.25 73.75) (end 209.0753 73.75) (width 0.25) (layer F.Cu) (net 2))
 (segment (start 208.6987 94.6763) (end 209.5 93.875) (width 0.25) (layer F.Cu) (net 13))
 (segment (start 224.05 96.75) (end 221.4912 99.3088) (width 0.25) (layer F.Cu) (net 13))
 (segment (start 221.4912 99.3088) (end 211.9924 99.3088) (width 0.25) (layer F.Cu) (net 13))
 (segment (start 211.9924 99.3088) (end 211.6236 98.94) (width 0.25) (layer F.Cu) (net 13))
 (segment (start 211.6236 98.94) (end 211.6236 97.747) (width 0.25) (layer F.Cu) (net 13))
 (segment (start 211.6236 97.747) (end 210.7631 96.8865) (width 0.25) (layer F.Cu) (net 13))
 (segment (start 210.7631 96.8865) (end 209.4065 96.8865) (width 0.25) (layer F.Cu) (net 13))
 (segment (start 209.4065 96.8865) (end 208.6987 96.1787) (width 0.25) (layer F.Cu) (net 13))
 (segment (start 208.6987 96.1787) (end 208.6987 94.6763) (width 0.25) (layer F.Cu) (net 13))
 (segment (start 206.25 94.0873) (end 208.1097 94.0873) (width 0.25) (layer F.Cu) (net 13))
 (segment (start 208.1097 94.0873) (end 208.6987 94.6763) (width 0.25) (layer F.Cu) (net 13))
 (segment (start 206.25 94.0873) (end 206.25 93.6747) (width 0.25) (layer F.Cu) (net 13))
 (segment (start 206.25 94.5) (end 206.25 94.0873) (width 0.25) (layer F.Cu) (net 13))
 (segment (start 226.5 96.75) (end 224.05 96.75) (width 0.25) (layer F.Cu) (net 13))
 (segment (start 205.875 91.75) (end 205.875 93.2997) (width 0.25) (layer F.Cu) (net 13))
 (segment (start 205.875 93.2997) (end 206.25 93.6747) (width 0.25) (layer F.Cu) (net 13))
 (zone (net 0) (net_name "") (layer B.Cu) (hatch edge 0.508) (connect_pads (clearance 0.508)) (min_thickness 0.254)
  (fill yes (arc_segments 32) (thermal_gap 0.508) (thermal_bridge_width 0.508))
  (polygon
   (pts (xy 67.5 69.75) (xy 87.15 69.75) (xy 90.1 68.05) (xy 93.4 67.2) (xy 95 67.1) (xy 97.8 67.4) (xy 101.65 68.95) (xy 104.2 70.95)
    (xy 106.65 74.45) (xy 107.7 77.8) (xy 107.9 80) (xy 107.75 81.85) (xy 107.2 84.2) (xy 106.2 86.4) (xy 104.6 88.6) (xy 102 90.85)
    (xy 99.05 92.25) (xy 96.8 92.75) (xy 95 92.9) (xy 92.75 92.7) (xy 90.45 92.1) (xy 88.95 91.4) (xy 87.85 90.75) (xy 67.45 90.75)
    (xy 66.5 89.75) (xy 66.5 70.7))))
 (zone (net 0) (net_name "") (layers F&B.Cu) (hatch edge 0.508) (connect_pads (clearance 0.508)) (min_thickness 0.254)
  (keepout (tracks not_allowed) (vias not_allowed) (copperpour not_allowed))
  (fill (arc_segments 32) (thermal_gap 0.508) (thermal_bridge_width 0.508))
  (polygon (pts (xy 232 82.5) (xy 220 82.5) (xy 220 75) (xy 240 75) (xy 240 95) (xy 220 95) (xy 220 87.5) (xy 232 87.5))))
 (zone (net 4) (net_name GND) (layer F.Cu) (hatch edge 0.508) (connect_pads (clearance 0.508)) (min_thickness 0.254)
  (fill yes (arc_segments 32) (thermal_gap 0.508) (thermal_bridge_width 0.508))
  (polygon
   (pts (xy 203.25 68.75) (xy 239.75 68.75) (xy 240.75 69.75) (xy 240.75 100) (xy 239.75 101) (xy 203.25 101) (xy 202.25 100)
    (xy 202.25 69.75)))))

